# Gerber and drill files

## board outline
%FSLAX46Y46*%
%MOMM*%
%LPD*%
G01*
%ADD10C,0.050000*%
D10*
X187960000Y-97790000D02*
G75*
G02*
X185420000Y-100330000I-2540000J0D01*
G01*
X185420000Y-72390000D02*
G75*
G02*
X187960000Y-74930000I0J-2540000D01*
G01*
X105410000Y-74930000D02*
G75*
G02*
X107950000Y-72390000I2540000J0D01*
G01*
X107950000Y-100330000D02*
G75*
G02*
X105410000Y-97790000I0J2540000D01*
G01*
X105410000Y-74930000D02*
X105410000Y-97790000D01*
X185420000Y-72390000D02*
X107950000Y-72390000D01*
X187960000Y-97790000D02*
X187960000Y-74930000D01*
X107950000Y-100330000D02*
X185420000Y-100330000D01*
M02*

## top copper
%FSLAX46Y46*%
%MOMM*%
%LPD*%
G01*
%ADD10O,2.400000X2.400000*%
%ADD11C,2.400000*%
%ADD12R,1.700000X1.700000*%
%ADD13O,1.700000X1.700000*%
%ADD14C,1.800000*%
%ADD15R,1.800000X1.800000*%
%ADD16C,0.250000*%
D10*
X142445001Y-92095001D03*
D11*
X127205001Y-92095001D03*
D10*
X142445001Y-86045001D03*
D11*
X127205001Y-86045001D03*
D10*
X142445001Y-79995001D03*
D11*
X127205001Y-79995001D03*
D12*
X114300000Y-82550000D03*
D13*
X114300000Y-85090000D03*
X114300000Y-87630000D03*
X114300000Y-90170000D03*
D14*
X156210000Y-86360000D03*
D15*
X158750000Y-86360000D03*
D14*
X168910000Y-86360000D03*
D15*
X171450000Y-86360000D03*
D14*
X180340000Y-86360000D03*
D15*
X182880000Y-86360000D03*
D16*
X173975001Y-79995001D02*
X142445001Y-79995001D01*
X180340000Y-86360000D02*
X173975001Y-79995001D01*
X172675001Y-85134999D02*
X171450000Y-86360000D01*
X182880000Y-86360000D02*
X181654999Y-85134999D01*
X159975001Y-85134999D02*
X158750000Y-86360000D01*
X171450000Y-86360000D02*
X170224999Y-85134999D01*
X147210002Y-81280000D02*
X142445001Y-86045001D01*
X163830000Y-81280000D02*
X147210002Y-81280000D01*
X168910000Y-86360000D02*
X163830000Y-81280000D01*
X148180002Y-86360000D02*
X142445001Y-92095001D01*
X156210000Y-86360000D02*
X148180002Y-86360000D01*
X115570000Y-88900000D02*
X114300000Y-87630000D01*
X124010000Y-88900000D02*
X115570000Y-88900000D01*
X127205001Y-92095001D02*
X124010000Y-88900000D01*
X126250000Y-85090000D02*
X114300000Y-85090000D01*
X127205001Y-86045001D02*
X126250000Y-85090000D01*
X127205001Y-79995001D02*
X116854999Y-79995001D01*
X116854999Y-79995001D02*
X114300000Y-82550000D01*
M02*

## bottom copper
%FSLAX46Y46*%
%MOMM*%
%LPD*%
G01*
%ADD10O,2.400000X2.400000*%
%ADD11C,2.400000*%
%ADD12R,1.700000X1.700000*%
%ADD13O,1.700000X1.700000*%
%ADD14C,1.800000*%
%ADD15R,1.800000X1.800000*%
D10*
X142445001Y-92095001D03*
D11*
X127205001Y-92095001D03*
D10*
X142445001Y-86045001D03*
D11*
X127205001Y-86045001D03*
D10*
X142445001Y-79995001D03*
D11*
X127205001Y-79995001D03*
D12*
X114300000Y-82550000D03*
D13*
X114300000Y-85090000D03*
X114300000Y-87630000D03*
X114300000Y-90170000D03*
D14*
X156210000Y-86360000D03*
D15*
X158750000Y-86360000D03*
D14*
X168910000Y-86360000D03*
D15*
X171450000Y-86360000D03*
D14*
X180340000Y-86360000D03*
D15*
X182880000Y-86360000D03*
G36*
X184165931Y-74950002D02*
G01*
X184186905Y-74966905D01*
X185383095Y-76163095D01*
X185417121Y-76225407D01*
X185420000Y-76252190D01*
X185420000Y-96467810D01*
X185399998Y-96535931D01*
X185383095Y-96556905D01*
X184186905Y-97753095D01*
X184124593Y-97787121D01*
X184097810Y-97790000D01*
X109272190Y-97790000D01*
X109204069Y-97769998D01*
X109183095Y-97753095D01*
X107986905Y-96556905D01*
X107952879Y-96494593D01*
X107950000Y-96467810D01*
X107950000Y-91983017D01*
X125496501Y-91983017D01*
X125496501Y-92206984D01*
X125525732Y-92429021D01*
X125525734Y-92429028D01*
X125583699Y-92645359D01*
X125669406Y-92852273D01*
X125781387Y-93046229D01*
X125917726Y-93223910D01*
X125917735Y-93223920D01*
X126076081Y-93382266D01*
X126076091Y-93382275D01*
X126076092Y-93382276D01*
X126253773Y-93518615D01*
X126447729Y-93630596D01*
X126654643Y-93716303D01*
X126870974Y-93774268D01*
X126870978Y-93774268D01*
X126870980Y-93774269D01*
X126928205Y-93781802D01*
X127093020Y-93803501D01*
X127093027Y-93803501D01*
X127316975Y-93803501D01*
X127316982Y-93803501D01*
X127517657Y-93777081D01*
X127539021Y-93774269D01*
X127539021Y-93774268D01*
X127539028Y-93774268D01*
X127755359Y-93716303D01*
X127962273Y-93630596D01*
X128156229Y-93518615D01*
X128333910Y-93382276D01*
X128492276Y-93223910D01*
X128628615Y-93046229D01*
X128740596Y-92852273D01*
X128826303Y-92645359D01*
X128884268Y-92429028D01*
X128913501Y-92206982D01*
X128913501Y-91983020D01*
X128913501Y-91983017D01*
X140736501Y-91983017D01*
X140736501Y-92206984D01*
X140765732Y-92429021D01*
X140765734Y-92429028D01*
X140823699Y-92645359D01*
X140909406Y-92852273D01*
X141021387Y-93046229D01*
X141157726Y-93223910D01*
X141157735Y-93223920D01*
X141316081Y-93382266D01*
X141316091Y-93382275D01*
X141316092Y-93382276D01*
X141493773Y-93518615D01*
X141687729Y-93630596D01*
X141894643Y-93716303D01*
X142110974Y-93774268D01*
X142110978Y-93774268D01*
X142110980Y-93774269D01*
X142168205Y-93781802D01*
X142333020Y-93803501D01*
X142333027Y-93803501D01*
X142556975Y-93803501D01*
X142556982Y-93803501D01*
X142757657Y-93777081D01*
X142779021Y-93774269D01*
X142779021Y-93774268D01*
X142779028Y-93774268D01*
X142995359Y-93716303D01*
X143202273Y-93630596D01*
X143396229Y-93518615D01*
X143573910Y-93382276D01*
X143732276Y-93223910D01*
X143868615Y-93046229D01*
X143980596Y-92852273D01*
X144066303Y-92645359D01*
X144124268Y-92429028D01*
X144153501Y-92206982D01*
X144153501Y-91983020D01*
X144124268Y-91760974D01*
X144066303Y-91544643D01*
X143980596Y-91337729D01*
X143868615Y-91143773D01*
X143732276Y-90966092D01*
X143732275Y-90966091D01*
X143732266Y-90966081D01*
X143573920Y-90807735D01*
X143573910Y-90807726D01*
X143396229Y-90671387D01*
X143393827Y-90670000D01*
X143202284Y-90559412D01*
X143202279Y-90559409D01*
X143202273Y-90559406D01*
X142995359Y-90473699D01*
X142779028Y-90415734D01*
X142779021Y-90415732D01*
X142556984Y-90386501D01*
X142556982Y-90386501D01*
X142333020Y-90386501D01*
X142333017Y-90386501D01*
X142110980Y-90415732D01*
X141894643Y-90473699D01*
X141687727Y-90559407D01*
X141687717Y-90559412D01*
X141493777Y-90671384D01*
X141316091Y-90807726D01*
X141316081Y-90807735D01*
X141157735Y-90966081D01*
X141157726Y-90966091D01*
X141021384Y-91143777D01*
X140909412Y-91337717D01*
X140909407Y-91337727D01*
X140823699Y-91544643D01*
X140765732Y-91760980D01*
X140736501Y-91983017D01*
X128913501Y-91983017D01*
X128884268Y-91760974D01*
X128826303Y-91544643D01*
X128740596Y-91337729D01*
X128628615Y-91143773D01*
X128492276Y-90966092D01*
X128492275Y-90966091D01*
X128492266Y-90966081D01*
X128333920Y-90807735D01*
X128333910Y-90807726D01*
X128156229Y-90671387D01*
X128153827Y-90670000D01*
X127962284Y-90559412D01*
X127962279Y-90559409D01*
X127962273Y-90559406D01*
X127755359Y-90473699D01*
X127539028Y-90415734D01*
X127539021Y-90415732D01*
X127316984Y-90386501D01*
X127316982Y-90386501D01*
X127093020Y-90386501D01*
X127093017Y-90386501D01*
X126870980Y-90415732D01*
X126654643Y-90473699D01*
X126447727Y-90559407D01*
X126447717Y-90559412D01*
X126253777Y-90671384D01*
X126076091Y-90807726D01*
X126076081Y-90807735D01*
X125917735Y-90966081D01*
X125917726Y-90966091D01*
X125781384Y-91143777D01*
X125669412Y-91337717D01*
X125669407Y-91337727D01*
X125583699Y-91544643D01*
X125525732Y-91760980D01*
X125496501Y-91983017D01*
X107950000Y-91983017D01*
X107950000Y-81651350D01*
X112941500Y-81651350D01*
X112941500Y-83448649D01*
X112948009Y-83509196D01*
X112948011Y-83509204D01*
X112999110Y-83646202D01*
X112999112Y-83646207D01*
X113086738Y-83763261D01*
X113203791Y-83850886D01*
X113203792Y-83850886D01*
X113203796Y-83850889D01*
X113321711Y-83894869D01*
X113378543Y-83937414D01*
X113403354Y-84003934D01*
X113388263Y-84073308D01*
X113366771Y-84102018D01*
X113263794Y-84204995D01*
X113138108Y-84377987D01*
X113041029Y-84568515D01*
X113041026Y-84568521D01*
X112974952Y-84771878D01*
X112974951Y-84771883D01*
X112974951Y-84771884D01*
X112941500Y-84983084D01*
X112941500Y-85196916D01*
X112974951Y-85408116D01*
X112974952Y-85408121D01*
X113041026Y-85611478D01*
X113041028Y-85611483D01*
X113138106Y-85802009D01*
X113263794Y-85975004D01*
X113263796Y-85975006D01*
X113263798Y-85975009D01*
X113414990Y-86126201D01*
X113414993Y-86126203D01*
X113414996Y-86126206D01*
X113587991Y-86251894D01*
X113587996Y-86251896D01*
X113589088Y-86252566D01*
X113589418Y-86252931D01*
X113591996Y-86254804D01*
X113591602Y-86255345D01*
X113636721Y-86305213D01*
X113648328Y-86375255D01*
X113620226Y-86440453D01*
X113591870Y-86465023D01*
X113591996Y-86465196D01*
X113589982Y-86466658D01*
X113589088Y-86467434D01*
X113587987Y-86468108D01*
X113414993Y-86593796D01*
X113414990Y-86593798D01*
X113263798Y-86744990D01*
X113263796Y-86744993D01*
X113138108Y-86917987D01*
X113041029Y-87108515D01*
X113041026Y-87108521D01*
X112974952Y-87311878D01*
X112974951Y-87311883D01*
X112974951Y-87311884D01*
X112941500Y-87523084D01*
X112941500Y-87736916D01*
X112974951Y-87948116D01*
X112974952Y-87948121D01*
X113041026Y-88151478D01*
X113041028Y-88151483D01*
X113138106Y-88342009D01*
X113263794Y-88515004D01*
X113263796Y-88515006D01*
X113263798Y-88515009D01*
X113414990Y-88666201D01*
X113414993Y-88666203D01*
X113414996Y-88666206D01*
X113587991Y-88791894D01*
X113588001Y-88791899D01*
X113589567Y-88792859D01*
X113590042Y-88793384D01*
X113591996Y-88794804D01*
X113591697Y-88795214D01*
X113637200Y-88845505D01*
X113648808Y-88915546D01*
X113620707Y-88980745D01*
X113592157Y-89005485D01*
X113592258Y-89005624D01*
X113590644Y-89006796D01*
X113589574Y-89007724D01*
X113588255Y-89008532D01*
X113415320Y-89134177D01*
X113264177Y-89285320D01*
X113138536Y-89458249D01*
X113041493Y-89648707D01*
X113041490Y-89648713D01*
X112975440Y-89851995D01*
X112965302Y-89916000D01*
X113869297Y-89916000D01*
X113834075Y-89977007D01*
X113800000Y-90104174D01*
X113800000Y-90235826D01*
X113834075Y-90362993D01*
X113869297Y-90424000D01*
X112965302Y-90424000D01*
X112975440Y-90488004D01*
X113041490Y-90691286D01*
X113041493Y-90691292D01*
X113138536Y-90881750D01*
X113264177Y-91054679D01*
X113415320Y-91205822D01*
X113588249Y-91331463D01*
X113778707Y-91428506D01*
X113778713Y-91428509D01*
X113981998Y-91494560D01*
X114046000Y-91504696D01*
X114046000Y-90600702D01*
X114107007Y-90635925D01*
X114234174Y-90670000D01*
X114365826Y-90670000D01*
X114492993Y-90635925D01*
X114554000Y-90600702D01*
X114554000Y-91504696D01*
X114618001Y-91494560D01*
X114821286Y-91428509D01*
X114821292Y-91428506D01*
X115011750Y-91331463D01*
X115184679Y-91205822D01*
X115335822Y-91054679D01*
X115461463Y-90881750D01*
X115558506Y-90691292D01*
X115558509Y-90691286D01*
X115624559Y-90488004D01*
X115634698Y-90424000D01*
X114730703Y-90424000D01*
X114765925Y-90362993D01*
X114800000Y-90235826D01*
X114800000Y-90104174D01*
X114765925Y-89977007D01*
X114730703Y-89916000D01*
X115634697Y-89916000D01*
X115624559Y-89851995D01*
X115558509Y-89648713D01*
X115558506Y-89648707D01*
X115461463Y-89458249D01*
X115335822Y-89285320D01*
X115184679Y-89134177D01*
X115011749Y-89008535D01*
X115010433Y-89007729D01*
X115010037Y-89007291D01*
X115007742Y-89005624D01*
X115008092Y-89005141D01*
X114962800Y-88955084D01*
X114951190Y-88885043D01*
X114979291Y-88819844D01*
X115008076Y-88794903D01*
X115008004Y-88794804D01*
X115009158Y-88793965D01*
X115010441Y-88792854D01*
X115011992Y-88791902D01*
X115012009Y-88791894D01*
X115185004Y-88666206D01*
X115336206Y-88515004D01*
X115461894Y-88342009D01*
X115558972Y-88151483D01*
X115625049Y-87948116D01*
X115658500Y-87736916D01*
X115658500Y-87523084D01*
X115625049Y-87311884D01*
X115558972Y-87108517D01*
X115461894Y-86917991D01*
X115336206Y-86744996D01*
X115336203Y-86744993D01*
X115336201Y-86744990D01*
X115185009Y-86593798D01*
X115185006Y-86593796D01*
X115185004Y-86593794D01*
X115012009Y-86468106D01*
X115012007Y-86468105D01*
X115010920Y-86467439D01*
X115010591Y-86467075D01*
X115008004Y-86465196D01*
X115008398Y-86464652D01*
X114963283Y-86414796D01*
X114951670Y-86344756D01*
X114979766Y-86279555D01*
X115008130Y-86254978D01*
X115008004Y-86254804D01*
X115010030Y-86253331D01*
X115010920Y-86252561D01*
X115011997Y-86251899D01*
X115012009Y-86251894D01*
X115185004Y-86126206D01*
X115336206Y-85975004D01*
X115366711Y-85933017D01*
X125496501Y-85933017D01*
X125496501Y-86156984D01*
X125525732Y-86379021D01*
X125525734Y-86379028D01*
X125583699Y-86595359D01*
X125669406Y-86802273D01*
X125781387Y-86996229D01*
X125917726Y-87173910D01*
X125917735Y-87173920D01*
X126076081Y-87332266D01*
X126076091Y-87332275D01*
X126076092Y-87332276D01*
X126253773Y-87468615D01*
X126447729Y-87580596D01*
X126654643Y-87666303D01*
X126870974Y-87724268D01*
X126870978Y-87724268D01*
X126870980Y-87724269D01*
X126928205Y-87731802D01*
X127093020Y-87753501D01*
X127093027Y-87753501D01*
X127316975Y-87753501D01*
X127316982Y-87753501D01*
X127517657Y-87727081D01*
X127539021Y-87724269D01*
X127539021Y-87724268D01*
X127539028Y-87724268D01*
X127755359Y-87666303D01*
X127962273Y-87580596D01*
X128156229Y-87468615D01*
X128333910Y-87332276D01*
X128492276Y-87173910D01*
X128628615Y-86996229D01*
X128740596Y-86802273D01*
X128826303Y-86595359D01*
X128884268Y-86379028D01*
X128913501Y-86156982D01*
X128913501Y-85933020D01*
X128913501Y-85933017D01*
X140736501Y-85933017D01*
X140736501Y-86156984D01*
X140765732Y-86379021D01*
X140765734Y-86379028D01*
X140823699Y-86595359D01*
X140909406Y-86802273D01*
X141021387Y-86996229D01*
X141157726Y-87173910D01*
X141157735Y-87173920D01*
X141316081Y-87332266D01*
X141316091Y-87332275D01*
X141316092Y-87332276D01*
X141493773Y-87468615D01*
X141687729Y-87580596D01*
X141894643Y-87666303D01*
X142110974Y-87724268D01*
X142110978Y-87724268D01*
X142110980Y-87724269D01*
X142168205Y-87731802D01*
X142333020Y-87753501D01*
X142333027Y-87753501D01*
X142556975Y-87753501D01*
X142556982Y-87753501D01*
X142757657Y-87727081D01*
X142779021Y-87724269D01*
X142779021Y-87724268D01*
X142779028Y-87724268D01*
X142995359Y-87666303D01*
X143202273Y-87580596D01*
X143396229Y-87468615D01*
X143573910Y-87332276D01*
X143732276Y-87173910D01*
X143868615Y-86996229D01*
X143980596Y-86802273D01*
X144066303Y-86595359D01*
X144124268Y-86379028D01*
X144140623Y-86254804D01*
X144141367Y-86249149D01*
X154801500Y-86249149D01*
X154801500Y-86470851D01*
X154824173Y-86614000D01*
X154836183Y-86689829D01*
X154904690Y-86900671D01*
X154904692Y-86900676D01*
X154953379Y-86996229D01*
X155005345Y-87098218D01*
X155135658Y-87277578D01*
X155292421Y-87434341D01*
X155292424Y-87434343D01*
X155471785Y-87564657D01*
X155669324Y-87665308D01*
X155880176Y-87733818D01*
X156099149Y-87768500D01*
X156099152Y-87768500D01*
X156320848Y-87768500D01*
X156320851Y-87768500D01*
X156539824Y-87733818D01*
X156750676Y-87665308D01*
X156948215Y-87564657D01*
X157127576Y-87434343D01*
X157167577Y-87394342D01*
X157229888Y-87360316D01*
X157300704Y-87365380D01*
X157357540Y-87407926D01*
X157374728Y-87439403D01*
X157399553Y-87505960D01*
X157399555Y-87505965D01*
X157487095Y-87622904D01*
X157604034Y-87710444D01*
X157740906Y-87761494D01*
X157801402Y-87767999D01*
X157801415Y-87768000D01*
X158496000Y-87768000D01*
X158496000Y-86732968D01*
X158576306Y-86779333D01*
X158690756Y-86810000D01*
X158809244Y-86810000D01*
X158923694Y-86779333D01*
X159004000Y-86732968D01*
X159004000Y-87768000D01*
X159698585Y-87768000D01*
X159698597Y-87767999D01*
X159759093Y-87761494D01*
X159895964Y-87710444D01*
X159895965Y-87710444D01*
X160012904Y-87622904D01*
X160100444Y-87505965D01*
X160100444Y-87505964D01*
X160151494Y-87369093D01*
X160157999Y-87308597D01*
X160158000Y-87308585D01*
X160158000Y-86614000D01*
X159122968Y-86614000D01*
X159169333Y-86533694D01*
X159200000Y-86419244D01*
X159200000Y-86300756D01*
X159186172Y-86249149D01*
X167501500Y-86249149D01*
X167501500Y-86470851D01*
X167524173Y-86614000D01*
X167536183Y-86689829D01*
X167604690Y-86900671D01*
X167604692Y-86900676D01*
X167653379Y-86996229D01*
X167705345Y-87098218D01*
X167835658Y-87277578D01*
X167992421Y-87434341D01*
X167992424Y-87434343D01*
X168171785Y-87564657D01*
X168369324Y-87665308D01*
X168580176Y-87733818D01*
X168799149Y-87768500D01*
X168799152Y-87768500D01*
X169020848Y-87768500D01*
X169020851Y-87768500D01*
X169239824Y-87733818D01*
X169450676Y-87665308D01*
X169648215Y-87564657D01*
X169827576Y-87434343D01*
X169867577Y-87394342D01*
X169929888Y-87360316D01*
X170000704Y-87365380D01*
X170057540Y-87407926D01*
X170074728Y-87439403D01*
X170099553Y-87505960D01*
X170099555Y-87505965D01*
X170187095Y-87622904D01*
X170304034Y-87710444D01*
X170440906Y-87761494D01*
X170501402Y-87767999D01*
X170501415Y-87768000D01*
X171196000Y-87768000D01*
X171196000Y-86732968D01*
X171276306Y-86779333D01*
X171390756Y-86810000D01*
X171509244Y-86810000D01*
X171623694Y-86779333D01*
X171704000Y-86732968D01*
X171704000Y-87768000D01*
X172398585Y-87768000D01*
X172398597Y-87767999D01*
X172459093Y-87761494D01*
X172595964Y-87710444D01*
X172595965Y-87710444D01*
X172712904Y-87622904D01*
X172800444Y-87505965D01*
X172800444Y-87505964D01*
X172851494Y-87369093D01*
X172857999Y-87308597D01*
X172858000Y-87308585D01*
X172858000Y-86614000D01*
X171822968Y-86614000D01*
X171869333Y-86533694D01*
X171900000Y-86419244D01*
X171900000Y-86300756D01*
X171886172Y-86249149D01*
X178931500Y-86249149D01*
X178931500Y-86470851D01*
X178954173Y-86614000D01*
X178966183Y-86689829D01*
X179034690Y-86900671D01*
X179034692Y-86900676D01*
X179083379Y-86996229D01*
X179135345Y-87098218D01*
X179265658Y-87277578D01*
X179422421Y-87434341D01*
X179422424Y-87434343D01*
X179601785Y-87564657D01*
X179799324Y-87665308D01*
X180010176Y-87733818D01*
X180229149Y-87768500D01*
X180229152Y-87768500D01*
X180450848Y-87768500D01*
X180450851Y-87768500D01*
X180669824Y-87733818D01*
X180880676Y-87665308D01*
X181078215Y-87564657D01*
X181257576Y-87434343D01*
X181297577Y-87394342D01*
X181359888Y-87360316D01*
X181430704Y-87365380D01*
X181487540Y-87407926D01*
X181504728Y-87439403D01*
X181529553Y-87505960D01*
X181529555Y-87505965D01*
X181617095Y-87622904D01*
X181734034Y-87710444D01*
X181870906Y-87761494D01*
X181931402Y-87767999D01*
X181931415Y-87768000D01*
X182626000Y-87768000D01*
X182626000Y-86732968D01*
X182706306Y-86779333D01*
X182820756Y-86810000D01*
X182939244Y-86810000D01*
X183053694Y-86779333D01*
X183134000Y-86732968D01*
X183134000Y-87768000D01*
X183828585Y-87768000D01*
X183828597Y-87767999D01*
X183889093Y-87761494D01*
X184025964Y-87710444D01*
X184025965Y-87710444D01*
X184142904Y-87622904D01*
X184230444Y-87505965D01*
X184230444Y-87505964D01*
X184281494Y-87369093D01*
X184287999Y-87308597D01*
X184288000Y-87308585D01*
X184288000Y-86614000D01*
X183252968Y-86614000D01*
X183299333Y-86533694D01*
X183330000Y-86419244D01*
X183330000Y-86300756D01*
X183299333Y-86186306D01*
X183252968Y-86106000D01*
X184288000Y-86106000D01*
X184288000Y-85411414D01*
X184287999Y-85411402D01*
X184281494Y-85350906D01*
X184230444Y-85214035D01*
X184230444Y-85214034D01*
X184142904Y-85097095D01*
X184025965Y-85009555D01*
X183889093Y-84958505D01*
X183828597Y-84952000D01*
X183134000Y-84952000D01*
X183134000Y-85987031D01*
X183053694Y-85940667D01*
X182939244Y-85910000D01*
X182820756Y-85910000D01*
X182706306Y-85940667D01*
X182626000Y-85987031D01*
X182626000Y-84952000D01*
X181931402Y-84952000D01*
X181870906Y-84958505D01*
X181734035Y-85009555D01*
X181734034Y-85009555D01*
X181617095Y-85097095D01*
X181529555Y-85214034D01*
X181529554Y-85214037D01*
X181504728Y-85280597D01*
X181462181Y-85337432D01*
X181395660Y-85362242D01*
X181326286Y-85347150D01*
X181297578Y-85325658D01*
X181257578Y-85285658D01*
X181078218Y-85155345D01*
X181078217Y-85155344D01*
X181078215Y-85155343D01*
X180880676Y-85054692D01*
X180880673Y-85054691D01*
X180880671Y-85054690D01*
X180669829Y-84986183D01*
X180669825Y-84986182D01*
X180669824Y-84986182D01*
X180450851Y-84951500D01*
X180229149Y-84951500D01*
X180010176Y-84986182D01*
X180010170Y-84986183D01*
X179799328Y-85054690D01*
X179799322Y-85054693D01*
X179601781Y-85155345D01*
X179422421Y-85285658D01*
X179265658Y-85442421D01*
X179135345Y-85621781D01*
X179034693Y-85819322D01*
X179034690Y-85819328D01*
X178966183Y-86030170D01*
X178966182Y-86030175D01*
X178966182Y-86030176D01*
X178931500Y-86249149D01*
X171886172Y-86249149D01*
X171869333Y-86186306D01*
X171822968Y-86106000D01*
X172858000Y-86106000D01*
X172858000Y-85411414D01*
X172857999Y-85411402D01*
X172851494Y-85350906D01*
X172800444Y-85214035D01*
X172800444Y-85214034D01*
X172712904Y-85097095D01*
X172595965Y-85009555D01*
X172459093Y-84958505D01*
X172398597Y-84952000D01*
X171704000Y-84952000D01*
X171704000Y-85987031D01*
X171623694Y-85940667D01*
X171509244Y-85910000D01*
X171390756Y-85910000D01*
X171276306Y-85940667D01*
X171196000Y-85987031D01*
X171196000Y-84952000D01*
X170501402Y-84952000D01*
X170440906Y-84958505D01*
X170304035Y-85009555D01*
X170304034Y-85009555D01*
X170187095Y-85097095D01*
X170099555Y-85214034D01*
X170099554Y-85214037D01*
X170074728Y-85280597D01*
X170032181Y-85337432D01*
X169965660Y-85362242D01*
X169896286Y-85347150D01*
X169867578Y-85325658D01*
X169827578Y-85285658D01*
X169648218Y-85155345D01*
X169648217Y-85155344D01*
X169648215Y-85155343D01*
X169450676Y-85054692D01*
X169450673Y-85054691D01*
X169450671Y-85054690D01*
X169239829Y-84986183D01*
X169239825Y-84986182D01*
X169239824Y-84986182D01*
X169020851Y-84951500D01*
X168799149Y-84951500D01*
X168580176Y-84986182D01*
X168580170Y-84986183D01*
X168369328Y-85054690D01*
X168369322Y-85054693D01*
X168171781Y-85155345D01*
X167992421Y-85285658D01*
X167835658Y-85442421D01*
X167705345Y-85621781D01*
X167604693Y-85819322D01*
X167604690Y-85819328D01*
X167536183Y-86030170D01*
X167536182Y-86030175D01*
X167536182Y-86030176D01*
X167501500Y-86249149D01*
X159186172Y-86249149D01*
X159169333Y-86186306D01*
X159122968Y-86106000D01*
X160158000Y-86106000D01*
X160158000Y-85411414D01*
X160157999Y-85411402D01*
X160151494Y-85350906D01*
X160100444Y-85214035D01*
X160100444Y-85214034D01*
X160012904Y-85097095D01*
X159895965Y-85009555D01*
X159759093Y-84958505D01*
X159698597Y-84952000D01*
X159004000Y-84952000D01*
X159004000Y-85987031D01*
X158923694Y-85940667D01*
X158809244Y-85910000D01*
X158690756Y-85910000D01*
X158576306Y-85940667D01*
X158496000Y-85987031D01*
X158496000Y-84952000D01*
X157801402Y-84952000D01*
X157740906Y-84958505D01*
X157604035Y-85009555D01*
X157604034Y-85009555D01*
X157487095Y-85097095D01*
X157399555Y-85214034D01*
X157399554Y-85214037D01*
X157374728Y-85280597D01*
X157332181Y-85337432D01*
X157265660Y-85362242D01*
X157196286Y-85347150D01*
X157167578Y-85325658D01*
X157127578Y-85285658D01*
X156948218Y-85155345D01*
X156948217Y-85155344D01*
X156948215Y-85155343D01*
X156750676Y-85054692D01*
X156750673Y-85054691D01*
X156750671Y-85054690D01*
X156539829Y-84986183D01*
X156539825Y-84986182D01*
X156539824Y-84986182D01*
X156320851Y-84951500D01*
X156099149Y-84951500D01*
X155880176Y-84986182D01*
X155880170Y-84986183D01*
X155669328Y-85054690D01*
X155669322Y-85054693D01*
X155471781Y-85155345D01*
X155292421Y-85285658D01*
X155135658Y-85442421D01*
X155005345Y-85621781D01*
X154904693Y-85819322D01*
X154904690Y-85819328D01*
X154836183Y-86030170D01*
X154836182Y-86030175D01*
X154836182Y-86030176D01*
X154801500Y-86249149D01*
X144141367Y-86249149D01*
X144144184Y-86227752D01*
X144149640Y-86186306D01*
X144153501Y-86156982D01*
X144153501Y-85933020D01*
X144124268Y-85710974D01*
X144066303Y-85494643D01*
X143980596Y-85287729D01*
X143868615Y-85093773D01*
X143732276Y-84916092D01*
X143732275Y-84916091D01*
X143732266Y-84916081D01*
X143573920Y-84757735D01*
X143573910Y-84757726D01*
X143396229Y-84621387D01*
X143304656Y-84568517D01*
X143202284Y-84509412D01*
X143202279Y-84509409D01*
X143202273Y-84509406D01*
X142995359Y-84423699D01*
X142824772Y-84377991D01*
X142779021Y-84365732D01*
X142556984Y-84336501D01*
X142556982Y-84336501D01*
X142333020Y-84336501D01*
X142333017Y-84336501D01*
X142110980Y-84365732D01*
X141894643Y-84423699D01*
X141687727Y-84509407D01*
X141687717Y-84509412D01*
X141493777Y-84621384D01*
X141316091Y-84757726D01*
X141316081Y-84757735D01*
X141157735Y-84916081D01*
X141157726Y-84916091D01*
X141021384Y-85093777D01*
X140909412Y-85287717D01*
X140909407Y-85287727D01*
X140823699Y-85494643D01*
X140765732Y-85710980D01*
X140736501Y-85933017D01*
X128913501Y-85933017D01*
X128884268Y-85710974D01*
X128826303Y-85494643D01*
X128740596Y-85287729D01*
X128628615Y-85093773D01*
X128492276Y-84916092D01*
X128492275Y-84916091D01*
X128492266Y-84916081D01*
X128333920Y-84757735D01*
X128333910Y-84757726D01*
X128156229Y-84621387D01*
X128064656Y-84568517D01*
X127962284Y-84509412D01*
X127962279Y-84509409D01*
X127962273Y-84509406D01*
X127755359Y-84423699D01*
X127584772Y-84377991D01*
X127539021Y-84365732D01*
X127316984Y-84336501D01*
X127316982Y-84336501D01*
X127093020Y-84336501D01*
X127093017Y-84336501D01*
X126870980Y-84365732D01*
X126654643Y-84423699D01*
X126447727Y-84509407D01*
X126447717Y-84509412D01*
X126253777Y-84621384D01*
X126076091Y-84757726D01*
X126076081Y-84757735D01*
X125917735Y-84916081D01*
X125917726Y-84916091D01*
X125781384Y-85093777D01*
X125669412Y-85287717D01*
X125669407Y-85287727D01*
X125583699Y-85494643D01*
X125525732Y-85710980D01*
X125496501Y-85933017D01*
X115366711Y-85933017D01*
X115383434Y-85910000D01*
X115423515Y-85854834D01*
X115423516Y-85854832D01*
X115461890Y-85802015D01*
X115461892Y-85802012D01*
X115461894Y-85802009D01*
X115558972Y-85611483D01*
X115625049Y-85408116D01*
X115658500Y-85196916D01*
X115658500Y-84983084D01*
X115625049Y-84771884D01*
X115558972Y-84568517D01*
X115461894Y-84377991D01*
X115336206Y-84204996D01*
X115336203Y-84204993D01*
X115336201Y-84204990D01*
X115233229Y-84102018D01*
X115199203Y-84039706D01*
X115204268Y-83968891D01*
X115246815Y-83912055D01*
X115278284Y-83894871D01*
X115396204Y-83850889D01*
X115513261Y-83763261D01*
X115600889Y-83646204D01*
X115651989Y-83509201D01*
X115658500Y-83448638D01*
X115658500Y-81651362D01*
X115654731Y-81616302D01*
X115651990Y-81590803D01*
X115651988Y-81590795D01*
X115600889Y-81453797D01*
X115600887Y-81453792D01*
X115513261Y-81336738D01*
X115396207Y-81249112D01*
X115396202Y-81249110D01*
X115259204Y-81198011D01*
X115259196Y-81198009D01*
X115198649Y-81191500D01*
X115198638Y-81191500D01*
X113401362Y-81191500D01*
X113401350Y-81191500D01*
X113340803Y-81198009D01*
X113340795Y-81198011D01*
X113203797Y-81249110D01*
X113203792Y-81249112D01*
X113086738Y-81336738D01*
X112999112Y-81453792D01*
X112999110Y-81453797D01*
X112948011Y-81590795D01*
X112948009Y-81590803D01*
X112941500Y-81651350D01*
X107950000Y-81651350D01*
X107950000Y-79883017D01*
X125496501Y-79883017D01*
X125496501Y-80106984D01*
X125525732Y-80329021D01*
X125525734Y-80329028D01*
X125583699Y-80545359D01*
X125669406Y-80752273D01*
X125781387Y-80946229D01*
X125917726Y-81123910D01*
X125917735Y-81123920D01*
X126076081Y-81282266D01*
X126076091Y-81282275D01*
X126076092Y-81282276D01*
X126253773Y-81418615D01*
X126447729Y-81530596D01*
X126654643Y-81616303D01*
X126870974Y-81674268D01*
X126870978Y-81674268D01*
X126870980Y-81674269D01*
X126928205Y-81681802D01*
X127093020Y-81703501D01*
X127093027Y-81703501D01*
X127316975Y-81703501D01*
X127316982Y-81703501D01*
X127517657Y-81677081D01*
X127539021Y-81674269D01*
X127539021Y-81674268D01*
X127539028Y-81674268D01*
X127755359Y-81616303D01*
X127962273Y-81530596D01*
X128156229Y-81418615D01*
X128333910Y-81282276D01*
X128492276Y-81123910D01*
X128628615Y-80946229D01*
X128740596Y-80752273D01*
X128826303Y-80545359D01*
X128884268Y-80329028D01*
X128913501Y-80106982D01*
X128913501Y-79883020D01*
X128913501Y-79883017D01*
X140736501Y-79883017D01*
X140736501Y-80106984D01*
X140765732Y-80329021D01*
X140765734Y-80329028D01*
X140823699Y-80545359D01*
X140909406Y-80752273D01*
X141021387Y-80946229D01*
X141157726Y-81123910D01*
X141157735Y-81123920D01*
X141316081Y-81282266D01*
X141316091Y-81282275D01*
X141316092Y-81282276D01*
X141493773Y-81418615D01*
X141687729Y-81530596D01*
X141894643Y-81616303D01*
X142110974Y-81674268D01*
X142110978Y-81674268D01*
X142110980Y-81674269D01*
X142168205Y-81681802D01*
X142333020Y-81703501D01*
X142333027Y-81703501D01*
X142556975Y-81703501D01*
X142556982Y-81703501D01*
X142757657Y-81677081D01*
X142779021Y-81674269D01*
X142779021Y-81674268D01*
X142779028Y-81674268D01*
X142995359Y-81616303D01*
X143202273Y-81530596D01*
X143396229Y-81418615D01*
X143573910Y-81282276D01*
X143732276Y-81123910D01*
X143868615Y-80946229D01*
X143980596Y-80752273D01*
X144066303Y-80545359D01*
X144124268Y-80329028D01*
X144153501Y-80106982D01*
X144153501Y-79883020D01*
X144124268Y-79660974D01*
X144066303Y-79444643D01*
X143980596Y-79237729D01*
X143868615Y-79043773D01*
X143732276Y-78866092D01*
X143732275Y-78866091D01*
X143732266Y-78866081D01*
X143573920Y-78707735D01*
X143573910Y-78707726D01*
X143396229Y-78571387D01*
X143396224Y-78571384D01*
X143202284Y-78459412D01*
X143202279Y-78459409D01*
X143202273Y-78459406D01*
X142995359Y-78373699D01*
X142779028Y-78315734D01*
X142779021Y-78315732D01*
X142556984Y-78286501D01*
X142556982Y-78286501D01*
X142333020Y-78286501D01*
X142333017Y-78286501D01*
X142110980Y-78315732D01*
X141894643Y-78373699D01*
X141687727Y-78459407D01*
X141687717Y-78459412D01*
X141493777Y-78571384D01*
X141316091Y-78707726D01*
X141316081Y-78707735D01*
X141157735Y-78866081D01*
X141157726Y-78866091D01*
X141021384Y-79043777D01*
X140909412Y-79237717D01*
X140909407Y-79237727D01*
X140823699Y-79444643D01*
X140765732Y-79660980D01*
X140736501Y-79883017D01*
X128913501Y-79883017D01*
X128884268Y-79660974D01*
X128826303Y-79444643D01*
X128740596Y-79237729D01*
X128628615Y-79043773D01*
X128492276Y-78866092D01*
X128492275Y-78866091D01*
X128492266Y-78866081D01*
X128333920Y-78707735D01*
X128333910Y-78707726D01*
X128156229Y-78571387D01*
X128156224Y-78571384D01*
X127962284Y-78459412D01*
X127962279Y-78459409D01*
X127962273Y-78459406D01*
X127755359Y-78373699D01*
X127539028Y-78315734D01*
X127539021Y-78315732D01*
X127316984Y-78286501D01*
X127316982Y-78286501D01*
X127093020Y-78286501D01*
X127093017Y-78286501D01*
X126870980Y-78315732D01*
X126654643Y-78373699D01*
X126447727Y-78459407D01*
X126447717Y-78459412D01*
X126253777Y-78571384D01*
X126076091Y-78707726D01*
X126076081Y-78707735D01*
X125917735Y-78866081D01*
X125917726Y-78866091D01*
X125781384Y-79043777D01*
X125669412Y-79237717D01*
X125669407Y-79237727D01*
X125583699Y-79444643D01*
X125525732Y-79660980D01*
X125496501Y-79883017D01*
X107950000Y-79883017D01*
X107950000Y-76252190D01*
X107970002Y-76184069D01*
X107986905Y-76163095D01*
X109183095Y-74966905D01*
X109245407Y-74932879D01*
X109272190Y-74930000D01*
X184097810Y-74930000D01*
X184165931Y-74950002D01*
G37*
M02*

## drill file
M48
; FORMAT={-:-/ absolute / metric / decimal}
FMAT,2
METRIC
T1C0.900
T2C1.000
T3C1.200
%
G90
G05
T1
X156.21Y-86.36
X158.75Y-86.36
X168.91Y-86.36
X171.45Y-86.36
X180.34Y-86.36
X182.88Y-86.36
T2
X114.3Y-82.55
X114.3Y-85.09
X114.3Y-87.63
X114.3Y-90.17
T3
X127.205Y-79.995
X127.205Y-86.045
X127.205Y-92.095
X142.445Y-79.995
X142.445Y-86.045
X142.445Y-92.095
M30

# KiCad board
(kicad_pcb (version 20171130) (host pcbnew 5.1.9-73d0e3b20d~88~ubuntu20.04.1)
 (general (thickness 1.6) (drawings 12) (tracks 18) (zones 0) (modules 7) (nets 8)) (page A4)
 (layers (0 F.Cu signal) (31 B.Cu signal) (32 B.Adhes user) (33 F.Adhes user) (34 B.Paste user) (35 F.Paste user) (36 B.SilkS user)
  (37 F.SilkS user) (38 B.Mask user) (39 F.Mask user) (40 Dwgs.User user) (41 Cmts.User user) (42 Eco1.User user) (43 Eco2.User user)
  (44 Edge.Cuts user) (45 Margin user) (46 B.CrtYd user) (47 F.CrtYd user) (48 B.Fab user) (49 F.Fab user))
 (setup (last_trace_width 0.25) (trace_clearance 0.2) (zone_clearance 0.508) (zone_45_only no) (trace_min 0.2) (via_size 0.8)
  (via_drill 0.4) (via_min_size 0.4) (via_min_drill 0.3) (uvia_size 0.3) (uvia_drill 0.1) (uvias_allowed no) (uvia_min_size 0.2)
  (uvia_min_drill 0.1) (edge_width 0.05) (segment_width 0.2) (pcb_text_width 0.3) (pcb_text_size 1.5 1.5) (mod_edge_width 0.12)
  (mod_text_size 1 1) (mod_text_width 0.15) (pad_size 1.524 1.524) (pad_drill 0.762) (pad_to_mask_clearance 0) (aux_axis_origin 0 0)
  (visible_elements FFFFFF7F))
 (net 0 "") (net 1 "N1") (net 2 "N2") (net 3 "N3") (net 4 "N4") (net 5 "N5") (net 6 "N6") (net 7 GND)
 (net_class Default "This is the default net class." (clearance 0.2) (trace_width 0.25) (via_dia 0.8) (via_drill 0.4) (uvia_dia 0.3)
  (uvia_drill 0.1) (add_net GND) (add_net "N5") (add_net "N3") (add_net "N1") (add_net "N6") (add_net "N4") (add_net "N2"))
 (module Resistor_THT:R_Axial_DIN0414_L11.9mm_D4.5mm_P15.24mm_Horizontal (layer F.Cu) (at 127.205001 92.095001)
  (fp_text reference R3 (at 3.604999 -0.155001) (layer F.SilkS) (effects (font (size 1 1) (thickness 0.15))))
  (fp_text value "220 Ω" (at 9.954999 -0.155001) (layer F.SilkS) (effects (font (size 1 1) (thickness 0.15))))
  (pad 2 thru_hole oval (at 15.24 0) (size 2.4 2.4) (drill 1.2) (layers *.Cu *.Mask) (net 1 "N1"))
  (pad 1 thru_hole circle (at 0 0) (size 2.4 2.4) (drill 1.2) (layers *.Cu *.Mask) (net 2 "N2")))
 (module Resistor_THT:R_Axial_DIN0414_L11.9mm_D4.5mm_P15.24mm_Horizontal (layer F.Cu) (at 127.205001 86.045001)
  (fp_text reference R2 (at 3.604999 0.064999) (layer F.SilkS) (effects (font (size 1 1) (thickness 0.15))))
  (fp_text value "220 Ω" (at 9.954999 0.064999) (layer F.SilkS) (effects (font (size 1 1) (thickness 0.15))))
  (pad 2 thru_hole oval (at 15.24 0) (size 2.4 2.4) (drill 1.2) (layers *.Cu *.Mask) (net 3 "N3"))
  (pad 1 thru_hole circle (at 0 0) (size 2.4 2.4) (drill 1.2) (layers *.Cu *.Mask) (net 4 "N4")))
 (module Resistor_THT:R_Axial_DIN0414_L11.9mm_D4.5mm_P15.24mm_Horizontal (layer F.Cu) (at 127.205001 79.995001)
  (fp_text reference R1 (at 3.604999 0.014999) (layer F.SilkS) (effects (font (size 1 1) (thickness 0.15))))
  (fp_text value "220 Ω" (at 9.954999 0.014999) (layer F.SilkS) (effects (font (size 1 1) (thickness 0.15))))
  (pad 2 thru_hole oval (at 15.24 0) (size 2.4 2.4) (drill 1.2) (layers *.Cu *.Mask) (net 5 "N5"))
  (pad 1 thru_hole circle (at 0 0) (size 2.4 2.4) (drill 1.2) (layers *.Cu *.Mask) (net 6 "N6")))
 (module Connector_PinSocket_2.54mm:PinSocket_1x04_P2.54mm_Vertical (layer F.Cu) (at 114.3 82.55)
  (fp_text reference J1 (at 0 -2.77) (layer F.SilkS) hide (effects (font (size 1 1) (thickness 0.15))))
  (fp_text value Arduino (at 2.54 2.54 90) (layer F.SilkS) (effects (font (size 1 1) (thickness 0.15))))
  (pad 1 thru_hole rect (at 0 0) (size 1.7 1.7) (drill 1) (layers *.Cu *.Mask) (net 6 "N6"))
  (pad 2 thru_hole oval (at 0 2.54) (size 1.7 1.7) (drill 1) (layers *.Cu *.Mask) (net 4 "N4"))
  (pad 3 thru_hole oval (at 0 5.08) (size 1.7 1.7) (drill 1) (layers *.Cu *.Mask) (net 2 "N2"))
  (pad 4 thru_hole oval (at 0 7.62) (size 1.7 1.7) (drill 1) (layers *.Cu *.Mask) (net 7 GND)))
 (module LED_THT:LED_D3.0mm (layer F.Cu) (at 158.75 86.36 180)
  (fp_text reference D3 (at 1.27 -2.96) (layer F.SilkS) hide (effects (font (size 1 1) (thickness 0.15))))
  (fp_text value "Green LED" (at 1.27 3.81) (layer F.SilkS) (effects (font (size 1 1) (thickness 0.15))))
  (pad 2 thru_hole circle (at 2.54 0 180) (size 1.8 1.8) (drill 0.9) (layers *.Cu *.Mask) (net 1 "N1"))
  (pad 1 thru_hole rect (at 0 0 180) (size 1.8 1.8) (drill 0.9) (layers *.Cu *.Mask) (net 7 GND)))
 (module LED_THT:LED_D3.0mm (layer F.Cu) (at 171.45 86.36 180)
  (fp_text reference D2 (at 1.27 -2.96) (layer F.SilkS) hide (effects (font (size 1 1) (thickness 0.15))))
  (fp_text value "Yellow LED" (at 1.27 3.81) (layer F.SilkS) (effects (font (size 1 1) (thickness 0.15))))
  (pad 2 thru_hole circle (at 2.54 0 180) (size 1.8 1.8) (drill 0.9) (layers *.Cu *.Mask) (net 3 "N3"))
  (pad 1 thru_hole rect (at 0 0 180) (size 1.8 1.8) (drill 0.9) (layers *.Cu *.Mask) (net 7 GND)))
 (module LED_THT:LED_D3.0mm (layer F.Cu) (at 182.88 86.36 180)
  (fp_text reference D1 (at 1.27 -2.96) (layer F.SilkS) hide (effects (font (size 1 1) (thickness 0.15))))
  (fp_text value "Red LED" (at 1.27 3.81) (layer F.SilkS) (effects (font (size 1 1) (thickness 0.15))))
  (pad 2 thru_hole circle (at 2.54 0 180) (size 1.8 1.8) (drill 0.9) (layers *.Cu *.Mask) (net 5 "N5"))
  (pad 1 thru_hole rect (at 0 0 180) (size 1.8 1.8) (drill 0.9) (layers *.Cu *.Mask) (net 7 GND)))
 (gr_arc (start 185.42 97.79) (end 185.42 100.33) (angle -90) (layer Edge.Cuts) (width 0.05))
 (gr_arc (start 185.42 74.93) (end 187.96 74.93) (angle -90) (layer Edge.Cuts) (width 0.05))
 (gr_arc (start 107.95 74.93) (end 107.95 72.39) (angle -90) (layer Edge.Cuts) (width 0.05))
 (gr_arc (start 107.95 97.79) (end 105.41 97.79) (angle -90) (layer Edge.Cuts) (width 0.05))
 (gr_line (start 105.41 74.93) (end 105.41 97.79) (layer Edge.Cuts) (width 0.05))
 (gr_line (start 185.42 72.39) (end 107.95 72.39) (layer Edge.Cuts) (width 0.05))
 (gr_line (start 187.96 97.79) (end 187.96 74.93) (layer Edge.Cuts) (width 0.05))
 (gr_line (start 107.95 100.33) (end 185.42 100.33) (layer Edge.Cuts) (width 0.05))
 (segment (start 173.975001 79.995001) (end 142.445001 79.995001) (width 0.25) (layer F.Cu) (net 5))
 (segment (start 180.34 86.36) (end 173.975001 79.995001) (width 0.25) (layer F.Cu) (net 5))
 (segment (start 172.675001 85.134999) (end 171.45 86.36) (width 0.25) (layer F.Cu) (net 7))
 (segment (start 182.88 86.36) (end 181.654999 85.134999) (width 0.25) (layer F.Cu) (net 7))
 (segment (start 159.975001 85.134999) (end 158.75 86.36) (width 0.25) (layer F.Cu) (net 7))
 (segment (start 171.45 86.36) (end 170.224999 85.134999) (width 0.25) (layer F.Cu) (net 7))
 (segment (start 147.210002 81.28) (end 142.445001 86.045001) (width 0.25) (layer F.Cu) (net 3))
 (segment (start 163.83 81.28) (end 147.210002 81.28) (width 0.25) (layer F.Cu) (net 3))
 (segment (start 168.91 86.36) (end 163.83 81.28) (width 0.25) (layer F.Cu) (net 3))
 (segment (start 148.180002 86.36) (end 142.445001 92.095001) (width 0.25) (layer F.Cu) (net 1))
 (segment (start 156.21 86.36) (end 148.180002 86.36) (width 0.25) (layer F.Cu) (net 1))
 (segment (start 115.57 88.9) (end 114.3 87.63) (width 0.25) (layer F.Cu) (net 2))
 (segment (start 124.01 88.9) (end 115.57 88.9) (width 0.25) (layer F.Cu) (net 2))
 (segment (start 127.205001 92.095001) (end 124.01 88.9) (width 0.25) (layer F.Cu) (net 2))
 (segment (start 126.25 85.09) (end 114.3 85.09) (width 0.25) (layer F.Cu) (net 4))
 (segment (start 127.205001 86.045001) (end 126.25 85.09) (width 0.25) (layer F.Cu) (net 4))
 (segment (start 127.205001 79.995001) (end 116.854999 79.995001) (width 0.25) (layer F.Cu) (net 6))
 (segment (start 116.854999 79.995001) (end 114.3 82.55) (width 0.25) (layer F.Cu) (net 6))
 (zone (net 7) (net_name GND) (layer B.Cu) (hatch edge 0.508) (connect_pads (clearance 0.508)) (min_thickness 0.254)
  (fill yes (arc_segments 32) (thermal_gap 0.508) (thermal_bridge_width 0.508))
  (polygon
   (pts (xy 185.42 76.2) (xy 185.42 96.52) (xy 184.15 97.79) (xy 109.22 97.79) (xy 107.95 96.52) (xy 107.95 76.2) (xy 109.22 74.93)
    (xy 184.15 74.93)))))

